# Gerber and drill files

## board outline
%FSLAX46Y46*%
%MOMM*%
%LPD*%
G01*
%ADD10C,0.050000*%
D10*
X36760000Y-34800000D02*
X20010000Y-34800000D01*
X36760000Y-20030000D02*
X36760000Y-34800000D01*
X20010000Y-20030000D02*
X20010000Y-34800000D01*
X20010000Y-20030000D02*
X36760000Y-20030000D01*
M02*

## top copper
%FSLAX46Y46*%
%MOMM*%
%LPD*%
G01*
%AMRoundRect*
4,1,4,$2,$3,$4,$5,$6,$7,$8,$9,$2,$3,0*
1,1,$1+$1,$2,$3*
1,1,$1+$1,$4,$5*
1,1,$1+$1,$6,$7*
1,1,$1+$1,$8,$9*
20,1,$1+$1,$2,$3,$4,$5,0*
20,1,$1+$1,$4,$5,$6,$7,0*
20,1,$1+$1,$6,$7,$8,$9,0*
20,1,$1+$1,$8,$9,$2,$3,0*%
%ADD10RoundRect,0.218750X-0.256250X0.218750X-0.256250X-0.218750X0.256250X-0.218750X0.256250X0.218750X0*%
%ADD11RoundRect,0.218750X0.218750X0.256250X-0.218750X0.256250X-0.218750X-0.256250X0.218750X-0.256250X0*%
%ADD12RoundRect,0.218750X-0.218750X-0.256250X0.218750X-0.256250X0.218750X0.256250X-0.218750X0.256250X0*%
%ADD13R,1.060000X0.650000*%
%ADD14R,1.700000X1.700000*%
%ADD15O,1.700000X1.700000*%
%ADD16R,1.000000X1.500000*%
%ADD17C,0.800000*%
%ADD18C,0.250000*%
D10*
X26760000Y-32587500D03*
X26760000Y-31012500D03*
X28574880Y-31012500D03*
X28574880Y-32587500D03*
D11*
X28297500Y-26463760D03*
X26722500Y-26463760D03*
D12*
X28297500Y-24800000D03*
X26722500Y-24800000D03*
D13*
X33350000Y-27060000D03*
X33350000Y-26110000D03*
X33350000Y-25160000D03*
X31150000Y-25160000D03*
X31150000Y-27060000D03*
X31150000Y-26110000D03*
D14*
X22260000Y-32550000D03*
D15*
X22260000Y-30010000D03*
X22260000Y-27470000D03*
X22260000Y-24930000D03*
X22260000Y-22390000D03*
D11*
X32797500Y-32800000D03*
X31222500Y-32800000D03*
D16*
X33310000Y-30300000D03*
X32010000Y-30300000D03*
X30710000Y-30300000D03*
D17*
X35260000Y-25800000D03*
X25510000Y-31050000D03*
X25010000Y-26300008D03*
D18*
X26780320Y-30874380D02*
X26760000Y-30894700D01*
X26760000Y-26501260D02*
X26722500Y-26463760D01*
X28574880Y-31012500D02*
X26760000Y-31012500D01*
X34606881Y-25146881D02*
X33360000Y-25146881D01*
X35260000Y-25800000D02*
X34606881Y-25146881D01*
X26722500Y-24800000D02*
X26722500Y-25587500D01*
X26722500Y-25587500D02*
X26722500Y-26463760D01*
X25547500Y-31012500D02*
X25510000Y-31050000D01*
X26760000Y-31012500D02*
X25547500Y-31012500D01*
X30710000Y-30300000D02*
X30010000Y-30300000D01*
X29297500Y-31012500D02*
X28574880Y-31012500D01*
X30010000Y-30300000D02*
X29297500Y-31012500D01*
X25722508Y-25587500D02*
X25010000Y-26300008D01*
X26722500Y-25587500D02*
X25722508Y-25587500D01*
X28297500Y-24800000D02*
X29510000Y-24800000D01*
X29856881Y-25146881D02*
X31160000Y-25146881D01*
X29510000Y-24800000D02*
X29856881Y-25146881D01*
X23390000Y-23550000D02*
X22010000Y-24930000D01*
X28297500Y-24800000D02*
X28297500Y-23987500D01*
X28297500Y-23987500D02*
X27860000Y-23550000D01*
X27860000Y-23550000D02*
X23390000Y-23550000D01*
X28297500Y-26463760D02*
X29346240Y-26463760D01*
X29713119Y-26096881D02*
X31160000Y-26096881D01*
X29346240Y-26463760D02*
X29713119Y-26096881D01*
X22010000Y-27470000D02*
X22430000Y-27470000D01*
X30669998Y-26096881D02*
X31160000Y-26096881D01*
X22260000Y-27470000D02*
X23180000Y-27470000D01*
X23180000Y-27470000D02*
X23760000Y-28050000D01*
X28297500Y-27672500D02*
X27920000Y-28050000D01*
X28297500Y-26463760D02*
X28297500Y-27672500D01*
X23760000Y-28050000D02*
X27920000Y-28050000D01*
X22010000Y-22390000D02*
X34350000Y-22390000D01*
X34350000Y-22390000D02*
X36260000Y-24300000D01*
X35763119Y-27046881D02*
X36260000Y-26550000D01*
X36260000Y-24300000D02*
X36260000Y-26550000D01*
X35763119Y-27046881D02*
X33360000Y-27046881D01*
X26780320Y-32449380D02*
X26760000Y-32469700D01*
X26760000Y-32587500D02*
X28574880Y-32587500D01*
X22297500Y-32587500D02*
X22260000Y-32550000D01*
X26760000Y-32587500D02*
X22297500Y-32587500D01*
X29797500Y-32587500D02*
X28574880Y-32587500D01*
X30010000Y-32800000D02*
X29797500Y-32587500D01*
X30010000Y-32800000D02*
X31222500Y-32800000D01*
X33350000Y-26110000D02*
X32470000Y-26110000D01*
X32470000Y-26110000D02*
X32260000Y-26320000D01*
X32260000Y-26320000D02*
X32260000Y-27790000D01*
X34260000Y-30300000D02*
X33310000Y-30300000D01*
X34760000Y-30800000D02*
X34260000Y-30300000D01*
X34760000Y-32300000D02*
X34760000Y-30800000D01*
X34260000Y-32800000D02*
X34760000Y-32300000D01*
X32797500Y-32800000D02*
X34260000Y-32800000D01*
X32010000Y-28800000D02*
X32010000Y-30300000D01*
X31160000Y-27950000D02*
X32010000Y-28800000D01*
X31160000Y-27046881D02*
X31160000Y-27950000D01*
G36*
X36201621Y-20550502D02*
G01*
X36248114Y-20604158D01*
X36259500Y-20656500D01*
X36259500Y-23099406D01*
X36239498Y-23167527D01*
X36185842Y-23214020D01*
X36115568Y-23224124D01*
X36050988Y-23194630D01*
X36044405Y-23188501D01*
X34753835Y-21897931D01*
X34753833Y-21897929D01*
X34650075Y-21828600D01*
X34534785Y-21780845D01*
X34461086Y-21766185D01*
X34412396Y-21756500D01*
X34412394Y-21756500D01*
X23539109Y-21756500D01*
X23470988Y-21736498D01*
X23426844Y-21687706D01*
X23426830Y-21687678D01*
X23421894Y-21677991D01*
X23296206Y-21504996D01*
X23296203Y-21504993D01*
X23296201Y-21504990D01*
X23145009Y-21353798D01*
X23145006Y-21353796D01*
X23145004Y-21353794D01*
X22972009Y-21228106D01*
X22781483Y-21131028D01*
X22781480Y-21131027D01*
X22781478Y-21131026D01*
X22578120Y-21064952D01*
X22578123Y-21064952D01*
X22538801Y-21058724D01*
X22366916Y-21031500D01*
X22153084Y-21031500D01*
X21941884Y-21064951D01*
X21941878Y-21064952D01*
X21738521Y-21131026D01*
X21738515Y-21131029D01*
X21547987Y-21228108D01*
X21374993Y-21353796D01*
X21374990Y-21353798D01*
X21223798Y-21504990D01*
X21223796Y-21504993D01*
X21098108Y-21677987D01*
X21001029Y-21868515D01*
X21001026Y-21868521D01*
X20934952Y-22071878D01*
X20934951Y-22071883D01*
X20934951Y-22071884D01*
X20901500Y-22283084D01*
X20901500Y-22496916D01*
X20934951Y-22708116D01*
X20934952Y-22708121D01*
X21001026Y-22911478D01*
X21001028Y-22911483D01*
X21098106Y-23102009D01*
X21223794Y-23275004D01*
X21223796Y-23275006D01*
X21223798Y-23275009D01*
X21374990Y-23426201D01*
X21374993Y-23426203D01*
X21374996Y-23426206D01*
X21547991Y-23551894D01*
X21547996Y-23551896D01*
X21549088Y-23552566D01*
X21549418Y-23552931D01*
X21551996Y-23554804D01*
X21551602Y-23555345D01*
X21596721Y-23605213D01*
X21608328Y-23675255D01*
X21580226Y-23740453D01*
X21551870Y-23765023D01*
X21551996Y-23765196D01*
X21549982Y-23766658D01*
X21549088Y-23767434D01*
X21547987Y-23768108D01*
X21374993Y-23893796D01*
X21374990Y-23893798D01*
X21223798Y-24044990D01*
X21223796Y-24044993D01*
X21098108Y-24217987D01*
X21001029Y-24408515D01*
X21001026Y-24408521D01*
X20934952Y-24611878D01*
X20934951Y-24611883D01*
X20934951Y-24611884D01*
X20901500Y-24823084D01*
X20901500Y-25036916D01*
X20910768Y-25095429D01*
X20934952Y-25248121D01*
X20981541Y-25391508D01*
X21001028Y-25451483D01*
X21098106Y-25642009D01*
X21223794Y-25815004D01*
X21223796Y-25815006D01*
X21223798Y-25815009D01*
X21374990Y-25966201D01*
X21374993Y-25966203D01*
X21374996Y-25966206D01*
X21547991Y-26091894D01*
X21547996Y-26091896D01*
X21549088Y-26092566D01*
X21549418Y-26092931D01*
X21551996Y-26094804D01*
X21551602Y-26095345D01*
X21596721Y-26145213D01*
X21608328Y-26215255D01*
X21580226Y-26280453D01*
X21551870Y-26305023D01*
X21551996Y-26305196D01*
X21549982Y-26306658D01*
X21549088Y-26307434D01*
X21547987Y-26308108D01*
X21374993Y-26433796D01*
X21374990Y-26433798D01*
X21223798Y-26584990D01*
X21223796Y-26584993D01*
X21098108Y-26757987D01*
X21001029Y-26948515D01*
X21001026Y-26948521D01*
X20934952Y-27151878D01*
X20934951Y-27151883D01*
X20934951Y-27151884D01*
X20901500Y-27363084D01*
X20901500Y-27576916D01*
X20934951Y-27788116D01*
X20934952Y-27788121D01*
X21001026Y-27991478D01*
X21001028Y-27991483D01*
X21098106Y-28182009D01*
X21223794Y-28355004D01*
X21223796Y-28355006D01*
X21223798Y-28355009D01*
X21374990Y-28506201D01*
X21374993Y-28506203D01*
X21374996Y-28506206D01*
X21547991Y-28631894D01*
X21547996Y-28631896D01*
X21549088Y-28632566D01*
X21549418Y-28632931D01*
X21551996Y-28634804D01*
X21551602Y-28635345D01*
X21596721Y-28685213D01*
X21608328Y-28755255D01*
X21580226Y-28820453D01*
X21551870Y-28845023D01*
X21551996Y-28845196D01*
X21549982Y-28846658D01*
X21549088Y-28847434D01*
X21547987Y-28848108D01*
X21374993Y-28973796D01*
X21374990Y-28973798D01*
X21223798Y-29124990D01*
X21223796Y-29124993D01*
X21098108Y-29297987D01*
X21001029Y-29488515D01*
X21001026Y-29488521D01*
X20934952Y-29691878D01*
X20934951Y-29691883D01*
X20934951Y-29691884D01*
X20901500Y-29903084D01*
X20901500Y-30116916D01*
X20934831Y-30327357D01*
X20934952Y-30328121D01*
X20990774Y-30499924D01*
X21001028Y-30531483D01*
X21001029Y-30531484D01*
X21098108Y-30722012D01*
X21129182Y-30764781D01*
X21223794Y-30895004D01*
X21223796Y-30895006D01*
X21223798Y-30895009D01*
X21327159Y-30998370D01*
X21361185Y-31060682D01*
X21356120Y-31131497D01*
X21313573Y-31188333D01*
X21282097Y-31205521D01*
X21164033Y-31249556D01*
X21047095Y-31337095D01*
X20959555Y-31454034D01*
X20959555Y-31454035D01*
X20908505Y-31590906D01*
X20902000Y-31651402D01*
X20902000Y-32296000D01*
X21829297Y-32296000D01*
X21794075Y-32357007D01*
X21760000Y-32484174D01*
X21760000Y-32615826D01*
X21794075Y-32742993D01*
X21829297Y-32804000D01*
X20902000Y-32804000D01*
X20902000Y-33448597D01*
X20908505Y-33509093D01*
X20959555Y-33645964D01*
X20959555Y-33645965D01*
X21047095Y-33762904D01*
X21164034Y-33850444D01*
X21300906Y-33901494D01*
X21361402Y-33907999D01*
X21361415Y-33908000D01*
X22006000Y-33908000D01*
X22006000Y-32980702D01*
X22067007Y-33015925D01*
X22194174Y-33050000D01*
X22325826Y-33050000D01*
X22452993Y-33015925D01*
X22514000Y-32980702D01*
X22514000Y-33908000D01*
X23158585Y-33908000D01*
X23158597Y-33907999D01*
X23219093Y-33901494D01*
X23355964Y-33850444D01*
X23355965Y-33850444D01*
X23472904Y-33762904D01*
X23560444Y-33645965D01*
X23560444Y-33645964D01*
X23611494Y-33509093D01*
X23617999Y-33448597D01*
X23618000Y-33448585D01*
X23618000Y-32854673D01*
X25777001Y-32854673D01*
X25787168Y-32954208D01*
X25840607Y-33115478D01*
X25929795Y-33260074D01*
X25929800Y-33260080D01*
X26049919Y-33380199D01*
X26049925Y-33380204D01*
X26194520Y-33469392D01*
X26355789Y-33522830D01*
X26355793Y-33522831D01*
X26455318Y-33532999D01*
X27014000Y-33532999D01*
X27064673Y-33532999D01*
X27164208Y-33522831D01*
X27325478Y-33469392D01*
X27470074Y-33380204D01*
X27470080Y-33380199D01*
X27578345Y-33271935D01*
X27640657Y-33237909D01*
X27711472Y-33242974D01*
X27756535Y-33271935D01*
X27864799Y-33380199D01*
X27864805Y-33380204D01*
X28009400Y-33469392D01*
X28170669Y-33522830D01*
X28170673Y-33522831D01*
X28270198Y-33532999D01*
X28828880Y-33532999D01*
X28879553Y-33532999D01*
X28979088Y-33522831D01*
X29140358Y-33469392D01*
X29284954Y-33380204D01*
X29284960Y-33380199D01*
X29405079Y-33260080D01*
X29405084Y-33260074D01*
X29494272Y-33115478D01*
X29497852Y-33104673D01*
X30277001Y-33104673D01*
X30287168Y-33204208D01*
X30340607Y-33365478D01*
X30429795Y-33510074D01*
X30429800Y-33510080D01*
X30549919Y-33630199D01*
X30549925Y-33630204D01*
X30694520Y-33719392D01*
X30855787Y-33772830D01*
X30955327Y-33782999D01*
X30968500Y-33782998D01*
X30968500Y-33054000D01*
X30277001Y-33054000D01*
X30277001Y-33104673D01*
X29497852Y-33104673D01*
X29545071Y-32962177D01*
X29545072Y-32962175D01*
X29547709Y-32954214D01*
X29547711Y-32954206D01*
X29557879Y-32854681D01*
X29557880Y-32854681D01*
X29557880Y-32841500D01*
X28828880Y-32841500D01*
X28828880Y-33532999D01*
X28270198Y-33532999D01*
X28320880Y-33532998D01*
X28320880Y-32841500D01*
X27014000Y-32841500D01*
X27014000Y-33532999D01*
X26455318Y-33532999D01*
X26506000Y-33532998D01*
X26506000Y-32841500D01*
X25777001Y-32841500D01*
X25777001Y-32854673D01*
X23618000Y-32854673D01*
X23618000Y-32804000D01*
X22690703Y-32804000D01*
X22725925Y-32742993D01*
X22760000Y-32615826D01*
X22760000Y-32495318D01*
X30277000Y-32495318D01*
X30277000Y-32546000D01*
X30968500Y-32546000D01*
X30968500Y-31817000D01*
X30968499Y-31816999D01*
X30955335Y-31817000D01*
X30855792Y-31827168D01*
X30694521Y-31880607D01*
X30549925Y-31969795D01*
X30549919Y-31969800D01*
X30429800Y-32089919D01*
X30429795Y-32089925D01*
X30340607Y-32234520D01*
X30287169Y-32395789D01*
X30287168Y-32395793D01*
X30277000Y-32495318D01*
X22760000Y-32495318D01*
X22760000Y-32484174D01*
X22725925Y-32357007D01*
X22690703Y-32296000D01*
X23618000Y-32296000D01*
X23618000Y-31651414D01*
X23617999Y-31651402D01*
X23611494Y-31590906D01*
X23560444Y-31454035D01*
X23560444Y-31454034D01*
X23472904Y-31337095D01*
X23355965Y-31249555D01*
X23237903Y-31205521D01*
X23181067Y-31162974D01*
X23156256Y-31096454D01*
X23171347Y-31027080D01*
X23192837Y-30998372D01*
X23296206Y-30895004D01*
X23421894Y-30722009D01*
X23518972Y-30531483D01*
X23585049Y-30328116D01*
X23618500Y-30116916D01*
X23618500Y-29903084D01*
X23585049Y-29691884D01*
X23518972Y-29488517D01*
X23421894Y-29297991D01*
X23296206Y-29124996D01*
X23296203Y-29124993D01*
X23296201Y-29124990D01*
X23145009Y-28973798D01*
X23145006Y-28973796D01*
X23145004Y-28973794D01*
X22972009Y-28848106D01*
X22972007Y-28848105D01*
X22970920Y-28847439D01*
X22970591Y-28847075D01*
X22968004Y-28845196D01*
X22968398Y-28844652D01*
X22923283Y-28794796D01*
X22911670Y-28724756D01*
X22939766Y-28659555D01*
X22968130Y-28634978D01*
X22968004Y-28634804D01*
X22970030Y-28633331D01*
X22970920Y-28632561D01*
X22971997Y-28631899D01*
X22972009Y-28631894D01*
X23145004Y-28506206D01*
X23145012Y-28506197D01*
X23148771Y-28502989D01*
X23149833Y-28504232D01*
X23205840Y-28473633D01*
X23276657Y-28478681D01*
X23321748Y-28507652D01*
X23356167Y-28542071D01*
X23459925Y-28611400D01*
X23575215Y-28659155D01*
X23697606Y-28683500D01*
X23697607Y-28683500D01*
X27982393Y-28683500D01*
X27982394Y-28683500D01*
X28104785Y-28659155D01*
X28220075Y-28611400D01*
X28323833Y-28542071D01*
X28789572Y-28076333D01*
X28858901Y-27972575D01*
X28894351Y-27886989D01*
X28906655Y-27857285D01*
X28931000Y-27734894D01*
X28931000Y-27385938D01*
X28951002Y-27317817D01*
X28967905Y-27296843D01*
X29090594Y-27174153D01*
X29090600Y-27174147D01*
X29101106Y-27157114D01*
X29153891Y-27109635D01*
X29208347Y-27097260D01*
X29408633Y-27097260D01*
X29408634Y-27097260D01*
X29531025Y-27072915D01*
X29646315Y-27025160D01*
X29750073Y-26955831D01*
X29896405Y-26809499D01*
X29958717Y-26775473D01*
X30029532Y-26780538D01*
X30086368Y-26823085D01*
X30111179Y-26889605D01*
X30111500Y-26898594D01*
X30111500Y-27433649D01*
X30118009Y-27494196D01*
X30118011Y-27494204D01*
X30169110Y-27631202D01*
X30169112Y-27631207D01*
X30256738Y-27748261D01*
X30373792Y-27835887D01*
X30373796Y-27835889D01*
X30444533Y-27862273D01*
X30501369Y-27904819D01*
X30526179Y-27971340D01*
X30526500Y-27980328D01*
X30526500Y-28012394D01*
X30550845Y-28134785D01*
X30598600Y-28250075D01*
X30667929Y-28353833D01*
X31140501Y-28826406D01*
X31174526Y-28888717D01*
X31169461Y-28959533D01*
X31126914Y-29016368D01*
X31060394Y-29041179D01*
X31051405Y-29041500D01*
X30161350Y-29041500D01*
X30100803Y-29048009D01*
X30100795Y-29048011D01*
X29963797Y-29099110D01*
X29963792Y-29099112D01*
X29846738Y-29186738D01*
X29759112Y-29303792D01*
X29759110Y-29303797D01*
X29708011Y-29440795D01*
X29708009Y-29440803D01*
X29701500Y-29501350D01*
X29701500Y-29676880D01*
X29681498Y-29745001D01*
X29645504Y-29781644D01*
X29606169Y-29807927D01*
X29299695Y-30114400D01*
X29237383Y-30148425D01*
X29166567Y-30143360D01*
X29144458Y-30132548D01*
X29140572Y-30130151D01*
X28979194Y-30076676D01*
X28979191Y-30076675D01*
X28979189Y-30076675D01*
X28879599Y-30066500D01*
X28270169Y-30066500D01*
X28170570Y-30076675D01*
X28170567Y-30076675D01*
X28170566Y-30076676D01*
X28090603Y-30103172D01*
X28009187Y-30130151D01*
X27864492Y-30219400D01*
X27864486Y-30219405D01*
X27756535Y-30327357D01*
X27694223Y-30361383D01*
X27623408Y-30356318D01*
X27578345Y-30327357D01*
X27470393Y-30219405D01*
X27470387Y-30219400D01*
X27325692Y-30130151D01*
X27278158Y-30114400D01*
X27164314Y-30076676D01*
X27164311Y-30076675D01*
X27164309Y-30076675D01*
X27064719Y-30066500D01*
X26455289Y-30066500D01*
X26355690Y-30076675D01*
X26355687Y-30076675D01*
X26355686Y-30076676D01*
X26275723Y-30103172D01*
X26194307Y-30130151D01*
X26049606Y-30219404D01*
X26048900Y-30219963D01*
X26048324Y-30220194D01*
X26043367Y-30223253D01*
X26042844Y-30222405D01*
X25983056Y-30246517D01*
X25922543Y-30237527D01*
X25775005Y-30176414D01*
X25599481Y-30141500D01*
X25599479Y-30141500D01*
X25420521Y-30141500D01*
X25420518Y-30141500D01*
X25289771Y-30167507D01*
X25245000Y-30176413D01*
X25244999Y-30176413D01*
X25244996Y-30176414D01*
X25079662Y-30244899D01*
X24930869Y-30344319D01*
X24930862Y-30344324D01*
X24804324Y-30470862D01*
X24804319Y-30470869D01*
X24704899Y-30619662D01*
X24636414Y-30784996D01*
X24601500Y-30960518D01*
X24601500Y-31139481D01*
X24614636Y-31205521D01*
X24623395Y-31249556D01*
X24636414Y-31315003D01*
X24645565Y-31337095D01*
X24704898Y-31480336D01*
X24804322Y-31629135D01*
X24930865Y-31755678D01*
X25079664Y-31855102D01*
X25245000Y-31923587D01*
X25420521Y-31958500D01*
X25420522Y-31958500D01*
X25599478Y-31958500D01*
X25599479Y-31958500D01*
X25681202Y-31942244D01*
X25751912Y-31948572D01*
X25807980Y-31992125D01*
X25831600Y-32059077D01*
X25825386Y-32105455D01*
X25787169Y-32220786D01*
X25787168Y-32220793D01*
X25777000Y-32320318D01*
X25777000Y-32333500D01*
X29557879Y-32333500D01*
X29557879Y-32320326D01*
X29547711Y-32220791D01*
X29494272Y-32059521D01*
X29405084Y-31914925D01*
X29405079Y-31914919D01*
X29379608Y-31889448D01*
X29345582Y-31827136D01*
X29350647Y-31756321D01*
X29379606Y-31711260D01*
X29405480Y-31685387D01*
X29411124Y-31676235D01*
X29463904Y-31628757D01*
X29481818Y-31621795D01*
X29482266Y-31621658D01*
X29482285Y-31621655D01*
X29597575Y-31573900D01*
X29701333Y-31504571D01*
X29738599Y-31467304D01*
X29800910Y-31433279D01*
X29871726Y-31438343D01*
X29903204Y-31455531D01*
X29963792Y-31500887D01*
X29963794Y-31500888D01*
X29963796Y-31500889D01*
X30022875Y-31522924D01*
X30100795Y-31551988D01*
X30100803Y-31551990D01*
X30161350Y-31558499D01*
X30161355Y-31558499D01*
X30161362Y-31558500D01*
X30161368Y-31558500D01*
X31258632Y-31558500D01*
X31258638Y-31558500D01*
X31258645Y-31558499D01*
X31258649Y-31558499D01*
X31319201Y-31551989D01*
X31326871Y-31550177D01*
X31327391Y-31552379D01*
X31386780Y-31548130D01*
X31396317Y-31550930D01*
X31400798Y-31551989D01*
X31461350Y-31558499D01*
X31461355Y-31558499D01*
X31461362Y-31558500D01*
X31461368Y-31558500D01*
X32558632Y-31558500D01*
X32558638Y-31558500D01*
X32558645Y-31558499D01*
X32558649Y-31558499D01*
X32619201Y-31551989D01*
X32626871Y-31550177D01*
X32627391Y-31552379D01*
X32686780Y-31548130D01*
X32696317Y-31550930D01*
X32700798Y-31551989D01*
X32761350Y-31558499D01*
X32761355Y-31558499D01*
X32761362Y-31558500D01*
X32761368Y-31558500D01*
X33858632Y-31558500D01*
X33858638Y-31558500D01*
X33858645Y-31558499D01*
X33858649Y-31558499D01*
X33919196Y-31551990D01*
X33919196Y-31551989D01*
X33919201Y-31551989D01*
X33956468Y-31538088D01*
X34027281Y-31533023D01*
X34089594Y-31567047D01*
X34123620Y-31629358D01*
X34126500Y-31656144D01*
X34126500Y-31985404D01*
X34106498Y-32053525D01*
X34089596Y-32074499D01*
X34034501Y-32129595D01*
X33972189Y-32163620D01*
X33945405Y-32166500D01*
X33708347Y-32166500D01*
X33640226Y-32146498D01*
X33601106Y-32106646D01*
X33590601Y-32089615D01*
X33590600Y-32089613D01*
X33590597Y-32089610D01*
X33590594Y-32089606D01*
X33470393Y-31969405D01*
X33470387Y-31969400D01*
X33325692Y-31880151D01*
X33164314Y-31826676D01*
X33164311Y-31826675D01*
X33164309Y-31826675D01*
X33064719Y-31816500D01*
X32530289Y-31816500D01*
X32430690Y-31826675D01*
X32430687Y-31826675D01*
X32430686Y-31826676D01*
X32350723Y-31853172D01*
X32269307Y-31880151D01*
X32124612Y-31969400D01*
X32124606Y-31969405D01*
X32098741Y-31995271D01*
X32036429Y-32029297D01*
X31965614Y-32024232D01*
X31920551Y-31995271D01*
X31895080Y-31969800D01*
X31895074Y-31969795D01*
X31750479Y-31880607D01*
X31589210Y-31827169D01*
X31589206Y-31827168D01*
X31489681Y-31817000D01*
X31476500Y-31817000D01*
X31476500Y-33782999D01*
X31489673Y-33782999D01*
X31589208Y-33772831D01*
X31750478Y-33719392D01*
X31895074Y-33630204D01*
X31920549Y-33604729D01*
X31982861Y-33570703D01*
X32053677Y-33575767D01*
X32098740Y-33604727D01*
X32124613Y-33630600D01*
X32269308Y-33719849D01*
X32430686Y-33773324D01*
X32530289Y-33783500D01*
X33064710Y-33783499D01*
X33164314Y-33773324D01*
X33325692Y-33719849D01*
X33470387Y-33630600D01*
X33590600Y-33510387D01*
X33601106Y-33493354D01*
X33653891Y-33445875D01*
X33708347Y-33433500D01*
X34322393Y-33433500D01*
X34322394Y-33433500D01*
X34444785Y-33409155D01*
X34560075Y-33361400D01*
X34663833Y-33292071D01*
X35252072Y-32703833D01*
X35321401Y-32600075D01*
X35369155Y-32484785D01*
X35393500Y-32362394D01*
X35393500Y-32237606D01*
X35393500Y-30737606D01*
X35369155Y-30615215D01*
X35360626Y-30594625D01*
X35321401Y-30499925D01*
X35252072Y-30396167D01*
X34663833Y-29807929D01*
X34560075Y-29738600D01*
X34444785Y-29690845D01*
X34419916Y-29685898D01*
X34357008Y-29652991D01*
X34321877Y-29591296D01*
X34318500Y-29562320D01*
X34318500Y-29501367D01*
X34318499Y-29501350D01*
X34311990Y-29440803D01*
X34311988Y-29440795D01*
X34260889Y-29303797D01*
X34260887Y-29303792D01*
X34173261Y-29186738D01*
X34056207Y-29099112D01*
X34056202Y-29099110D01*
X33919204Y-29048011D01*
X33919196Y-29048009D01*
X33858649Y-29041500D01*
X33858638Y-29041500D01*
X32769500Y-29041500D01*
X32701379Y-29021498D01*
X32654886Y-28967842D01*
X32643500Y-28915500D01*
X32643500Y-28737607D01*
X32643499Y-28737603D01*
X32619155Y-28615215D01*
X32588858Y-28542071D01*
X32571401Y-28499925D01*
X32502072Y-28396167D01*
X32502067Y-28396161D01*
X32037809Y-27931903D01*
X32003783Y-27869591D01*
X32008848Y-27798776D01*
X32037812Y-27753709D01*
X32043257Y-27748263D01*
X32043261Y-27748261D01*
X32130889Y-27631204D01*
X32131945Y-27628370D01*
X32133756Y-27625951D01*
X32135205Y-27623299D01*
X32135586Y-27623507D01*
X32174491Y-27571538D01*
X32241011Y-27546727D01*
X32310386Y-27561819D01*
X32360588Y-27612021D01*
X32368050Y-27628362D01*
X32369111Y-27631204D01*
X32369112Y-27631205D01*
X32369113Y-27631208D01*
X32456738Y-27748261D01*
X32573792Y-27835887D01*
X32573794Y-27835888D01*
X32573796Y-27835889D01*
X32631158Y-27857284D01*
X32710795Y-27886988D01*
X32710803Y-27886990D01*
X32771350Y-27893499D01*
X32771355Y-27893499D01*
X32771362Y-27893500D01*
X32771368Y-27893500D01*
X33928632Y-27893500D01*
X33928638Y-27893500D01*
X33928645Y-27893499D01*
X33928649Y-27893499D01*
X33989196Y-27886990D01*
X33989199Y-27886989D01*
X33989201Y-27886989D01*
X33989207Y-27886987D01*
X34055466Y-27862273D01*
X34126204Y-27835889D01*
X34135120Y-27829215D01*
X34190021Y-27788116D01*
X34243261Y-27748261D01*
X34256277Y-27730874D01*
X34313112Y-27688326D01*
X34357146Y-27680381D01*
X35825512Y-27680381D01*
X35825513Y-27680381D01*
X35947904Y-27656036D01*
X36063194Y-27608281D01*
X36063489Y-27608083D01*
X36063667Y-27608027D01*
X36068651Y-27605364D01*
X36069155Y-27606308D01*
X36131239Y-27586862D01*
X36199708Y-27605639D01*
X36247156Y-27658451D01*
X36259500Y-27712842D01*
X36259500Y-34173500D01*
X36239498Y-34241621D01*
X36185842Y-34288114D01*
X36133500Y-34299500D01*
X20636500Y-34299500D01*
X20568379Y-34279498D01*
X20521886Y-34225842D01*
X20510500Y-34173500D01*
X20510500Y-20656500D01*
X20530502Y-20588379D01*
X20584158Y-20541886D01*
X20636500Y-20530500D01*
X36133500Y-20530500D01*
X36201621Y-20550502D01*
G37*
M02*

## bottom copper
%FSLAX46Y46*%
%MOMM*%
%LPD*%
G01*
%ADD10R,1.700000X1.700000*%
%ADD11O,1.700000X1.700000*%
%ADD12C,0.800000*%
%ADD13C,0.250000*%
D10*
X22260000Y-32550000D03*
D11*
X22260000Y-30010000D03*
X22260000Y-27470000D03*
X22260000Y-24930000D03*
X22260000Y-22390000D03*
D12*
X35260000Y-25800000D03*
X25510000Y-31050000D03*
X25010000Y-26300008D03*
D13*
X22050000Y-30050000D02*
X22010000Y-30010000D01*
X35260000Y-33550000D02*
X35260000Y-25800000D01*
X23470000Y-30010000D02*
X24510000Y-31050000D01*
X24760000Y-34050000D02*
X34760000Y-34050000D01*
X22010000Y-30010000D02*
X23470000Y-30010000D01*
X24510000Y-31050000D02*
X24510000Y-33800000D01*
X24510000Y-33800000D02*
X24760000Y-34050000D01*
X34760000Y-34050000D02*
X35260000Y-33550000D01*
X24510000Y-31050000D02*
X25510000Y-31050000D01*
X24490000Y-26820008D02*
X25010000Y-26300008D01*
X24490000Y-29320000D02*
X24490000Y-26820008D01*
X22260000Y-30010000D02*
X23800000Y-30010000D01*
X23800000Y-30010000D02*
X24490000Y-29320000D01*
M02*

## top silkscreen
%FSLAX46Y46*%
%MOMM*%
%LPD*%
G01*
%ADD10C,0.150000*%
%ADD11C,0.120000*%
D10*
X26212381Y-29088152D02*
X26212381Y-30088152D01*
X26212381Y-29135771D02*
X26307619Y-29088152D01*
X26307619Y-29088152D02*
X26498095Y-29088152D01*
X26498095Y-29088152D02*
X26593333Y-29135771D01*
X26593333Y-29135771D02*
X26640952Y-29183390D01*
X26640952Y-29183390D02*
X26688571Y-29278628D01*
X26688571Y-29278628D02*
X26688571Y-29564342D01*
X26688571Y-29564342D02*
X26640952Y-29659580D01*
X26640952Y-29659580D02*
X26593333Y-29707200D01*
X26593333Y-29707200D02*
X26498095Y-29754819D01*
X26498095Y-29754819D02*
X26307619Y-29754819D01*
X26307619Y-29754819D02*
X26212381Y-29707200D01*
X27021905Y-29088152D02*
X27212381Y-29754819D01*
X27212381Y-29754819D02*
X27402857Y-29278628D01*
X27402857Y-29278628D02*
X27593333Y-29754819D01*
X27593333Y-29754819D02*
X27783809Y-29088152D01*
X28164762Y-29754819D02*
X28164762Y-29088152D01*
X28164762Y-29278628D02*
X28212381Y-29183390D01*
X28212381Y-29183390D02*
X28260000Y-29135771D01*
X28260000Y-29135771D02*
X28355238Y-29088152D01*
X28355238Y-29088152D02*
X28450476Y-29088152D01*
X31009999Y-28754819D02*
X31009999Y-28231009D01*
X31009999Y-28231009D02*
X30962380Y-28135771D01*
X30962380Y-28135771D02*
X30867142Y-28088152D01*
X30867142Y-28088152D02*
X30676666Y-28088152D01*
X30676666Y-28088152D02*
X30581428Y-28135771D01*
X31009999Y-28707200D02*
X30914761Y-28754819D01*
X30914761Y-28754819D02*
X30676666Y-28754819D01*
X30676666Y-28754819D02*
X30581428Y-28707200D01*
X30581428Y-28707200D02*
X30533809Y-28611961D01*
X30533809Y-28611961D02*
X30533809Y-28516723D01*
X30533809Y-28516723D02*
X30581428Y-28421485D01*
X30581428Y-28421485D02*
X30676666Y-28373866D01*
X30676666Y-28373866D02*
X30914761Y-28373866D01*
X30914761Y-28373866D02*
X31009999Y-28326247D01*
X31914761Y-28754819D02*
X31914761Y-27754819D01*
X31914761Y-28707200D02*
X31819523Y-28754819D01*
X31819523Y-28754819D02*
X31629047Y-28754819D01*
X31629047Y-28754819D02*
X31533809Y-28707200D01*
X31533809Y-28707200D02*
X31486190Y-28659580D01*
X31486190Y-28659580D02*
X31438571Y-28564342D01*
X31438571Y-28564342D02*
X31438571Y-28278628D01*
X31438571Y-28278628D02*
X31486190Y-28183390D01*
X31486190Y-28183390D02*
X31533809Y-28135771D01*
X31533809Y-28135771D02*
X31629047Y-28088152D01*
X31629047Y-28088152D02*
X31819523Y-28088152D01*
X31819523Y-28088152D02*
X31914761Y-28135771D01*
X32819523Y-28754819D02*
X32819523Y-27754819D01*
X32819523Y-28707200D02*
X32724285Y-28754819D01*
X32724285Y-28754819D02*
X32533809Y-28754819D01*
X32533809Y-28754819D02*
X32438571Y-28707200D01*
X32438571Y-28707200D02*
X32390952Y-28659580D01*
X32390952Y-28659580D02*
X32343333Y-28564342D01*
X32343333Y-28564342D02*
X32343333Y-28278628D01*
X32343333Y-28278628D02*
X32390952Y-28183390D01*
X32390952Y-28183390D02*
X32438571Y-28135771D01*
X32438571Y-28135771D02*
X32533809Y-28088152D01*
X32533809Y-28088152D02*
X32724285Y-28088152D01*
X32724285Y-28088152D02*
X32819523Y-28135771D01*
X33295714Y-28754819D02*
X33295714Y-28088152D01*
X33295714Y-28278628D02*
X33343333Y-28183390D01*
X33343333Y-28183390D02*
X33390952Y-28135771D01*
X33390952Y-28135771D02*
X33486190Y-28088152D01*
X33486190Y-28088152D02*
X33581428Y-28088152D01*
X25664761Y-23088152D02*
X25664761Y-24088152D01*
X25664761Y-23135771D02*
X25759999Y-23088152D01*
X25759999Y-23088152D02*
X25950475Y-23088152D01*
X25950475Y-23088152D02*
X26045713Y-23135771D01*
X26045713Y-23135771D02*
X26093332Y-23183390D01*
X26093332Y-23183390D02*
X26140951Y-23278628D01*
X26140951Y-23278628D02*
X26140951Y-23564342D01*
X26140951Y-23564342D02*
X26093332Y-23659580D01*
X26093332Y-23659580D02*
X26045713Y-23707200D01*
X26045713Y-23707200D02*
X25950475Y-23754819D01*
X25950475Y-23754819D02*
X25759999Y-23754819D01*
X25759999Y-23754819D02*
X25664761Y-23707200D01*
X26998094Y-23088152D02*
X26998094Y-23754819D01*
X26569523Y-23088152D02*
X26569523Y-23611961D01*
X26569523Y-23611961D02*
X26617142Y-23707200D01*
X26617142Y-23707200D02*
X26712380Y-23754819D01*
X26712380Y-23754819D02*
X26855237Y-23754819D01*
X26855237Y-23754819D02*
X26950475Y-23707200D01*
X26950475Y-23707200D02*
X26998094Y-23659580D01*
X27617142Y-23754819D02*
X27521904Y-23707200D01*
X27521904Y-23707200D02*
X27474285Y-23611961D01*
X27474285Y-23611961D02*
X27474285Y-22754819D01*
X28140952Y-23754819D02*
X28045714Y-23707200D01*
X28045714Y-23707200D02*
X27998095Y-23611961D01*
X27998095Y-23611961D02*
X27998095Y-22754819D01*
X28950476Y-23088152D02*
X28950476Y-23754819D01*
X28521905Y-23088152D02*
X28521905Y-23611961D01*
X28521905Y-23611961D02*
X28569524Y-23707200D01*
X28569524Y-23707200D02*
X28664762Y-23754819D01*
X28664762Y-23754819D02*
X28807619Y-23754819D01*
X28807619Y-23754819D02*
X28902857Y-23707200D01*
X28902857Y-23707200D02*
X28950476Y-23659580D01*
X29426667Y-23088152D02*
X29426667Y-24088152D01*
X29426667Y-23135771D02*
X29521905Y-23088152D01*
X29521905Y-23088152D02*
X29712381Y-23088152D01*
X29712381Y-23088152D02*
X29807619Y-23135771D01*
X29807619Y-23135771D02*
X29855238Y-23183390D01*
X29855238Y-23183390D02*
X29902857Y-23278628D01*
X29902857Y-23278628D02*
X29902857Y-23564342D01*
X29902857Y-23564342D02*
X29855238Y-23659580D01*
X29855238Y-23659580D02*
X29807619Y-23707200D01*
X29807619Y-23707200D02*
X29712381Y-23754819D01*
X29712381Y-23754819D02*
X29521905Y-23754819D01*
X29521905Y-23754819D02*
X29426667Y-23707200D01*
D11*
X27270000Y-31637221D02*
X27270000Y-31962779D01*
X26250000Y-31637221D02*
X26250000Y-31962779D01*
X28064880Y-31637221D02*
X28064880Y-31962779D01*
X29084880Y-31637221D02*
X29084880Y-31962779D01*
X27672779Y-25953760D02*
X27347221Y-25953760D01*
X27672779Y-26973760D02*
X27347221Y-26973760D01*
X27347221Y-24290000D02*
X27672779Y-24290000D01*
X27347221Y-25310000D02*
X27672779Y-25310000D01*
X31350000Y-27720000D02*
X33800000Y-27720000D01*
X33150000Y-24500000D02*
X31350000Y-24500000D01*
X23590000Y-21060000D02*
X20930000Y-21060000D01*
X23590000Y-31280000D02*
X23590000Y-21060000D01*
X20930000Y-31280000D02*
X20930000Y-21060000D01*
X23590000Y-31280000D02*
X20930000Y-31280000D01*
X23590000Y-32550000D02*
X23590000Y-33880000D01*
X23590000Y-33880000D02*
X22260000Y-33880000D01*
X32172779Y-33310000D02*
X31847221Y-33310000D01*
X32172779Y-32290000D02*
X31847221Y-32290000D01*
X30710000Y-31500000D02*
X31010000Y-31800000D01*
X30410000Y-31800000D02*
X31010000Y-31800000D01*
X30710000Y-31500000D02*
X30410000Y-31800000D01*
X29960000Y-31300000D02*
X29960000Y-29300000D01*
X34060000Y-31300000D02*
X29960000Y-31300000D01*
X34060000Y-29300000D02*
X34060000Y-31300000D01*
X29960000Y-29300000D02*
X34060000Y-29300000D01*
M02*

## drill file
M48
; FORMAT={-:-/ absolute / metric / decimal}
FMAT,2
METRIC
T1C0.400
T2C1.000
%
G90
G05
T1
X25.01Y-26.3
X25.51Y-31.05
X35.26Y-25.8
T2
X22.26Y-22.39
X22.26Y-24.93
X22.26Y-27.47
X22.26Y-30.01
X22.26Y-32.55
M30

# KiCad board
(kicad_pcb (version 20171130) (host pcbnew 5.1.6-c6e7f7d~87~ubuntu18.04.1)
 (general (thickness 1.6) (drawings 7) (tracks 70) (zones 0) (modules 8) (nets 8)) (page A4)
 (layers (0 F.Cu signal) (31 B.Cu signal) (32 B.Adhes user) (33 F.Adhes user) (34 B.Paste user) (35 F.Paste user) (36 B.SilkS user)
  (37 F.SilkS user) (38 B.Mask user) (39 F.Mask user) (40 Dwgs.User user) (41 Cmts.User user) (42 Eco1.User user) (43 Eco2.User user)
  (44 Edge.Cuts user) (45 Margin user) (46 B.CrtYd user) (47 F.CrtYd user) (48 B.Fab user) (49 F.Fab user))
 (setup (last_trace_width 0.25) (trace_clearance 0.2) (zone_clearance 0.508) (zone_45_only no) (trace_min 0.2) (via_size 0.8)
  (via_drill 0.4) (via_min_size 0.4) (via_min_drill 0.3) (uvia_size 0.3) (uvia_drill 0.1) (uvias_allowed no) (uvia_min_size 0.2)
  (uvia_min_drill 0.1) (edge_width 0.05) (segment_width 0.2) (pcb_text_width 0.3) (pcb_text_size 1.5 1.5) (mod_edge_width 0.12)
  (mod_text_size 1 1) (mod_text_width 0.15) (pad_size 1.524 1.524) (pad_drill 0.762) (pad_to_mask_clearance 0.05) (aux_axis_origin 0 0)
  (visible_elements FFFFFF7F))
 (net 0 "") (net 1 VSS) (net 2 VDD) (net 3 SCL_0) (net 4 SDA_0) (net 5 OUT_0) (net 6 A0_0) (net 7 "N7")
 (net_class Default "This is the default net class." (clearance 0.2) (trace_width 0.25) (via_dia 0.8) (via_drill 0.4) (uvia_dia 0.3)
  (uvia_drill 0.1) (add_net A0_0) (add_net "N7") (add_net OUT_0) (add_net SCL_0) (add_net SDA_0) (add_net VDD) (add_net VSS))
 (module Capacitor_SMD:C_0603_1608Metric (layer F.Cu) (at 26.76 31.8 270)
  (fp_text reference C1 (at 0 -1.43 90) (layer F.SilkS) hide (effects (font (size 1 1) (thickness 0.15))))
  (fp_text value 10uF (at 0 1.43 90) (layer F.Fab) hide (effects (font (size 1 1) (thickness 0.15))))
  (fp_line (start -0.162779 -0.51) (end 0.162779 -0.51) (layer F.SilkS) (width 0.12))
  (fp_line (start -0.162779 0.51) (end 0.162779 0.51) (layer F.SilkS) (width 0.12))
  (pad 2 smd roundrect (at 0.7875 0 270) (size 0.875 0.95) (layers F.Cu F.Paste F.Mask) (roundrect_rratio 0.25) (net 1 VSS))
  (pad 1 smd roundrect (at -0.7875 0 270) (size 0.875 0.95) (layers F.Cu F.Paste F.Mask) (roundrect_rratio 0.25) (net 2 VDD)))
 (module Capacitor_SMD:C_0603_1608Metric (layer F.Cu) (at 28.57488 31.8 270)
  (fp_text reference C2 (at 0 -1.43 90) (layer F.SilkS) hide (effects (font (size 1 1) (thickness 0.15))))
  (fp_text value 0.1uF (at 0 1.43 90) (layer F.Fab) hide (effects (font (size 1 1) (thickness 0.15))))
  (fp_line (start -0.162779 0.51) (end 0.162779 0.51) (layer F.SilkS) (width 0.12))
  (fp_line (start -0.162779 -0.51) (end 0.162779 -0.51) (layer F.SilkS) (width 0.12))
  (pad 1 smd roundrect (at -0.7875 0 270) (size 0.875 0.95) (layers F.Cu F.Paste F.Mask) (roundrect_rratio 0.25) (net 2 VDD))
  (pad 2 smd roundrect (at 0.7875 0 270) (size 0.875 0.95) (layers F.Cu F.Paste F.Mask) (roundrect_rratio 0.25) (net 1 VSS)))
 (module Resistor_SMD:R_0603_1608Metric (layer F.Cu) (at 27.51 26.46376 180)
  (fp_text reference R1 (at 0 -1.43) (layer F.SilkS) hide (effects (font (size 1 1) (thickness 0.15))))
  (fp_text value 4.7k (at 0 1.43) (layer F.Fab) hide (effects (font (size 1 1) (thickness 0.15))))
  (fp_line (start -0.162779 0.51) (end 0.162779 0.51) (layer F.SilkS) (width 0.12))
  (fp_line (start -0.162779 -0.51) (end 0.162779 -0.51) (layer F.SilkS) (width 0.12))
  (pad 1 smd roundrect (at -0.7875 0 180) (size 0.875 0.95) (layers F.Cu F.Paste F.Mask) (roundrect_rratio 0.25) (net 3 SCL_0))
  (pad 2 smd roundrect (at 0.7875 0 180) (size 0.875 0.95) (layers F.Cu F.Paste F.Mask) (roundrect_rratio 0.25) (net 2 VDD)))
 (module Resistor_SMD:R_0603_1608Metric (layer F.Cu) (at 27.51 24.8)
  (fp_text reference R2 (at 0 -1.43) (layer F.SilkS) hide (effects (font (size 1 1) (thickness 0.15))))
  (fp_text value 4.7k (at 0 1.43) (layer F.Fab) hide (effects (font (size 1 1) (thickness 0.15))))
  (fp_line (start -0.162779 -0.51) (end 0.162779 -0.51) (layer F.SilkS) (width 0.12))
  (fp_line (start -0.162779 0.51) (end 0.162779 0.51) (layer F.SilkS) (width 0.12))
  (pad 2 smd roundrect (at 0.7875 0) (size 0.875 0.95) (layers F.Cu F.Paste F.Mask) (roundrect_rratio 0.25) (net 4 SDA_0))
  (pad 1 smd roundrect (at -0.7875 0) (size 0.875 0.95) (layers F.Cu F.Paste F.Mask) (roundrect_rratio 0.25) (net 2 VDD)))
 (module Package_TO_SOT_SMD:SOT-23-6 (layer F.Cu) (at 32.25 26.11 180)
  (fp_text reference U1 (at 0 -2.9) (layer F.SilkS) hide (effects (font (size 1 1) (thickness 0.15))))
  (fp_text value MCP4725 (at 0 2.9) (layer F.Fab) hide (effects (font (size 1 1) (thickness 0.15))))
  (fp_line (start 0.9 -1.61) (end -1.55 -1.61) (layer F.SilkS) (width 0.12))
  (fp_line (start -0.9 1.61) (end 0.9 1.61) (layer F.SilkS) (width 0.12))
  (pad 1 smd rect (at -1.1 -0.95 180) (size 1.06 0.65) (layers F.Cu F.Paste F.Mask) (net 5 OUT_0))
  (pad 2 smd rect (at -1.1 0 180) (size 1.06 0.65) (layers F.Cu F.Paste F.Mask) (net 1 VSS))
  (pad 3 smd rect (at -1.1 0.95 180) (size 1.06 0.65) (layers F.Cu F.Paste F.Mask) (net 2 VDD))
  (pad 4 smd rect (at 1.1 0.95 180) (size 1.06 0.65) (layers F.Cu F.Paste F.Mask) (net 4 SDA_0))
  (pad 6 smd rect (at 1.1 -0.95 180) (size 1.06 0.65) (layers F.Cu F.Paste F.Mask) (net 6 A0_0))
  (pad 5 smd rect (at 1.1 0 180) (size 1.06 0.65) (layers F.Cu F.Paste F.Mask) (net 3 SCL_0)))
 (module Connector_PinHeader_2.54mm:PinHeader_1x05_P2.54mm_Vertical (layer F.Cu) (at 22.26 32.55 180)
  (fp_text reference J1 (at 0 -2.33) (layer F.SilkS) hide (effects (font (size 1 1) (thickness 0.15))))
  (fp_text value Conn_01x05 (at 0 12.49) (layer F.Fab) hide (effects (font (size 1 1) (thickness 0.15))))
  (fp_line (start -1.33 11.49) (end 1.33 11.49) (layer F.SilkS) (width 0.12))
  (fp_line (start -1.33 1.27) (end -1.33 11.49) (layer F.SilkS) (width 0.12))
  (fp_line (start 1.33 1.27) (end 1.33 11.49) (layer F.SilkS) (width 0.12))
  (fp_line (start -1.33 1.27) (end 1.33 1.27) (layer F.SilkS) (width 0.12))
  (fp_line (start -1.33 0) (end -1.33 -1.33) (layer F.SilkS) (width 0.12))
  (fp_line (start -1.33 -1.33) (end 0 -1.33) (layer F.SilkS) (width 0.12))
  (pad 1 thru_hole rect (at 0 0 180) (size 1.7 1.7) (drill 1) (layers *.Cu *.Mask) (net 1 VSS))
  (pad 2 thru_hole oval (at 0 2.54 180) (size 1.7 1.7) (drill 1) (layers *.Cu *.Mask) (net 2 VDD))
  (pad 3 thru_hole oval (at 0 5.08 180) (size 1.7 1.7) (drill 1) (layers *.Cu *.Mask) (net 3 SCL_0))
  (pad 4 thru_hole oval (at 0 7.62 180) (size 1.7 1.7) (drill 1) (layers *.Cu *.Mask) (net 4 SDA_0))
  (pad 5 thru_hole oval (at 0 10.16 180) (size 1.7 1.7) (drill 1) (layers *.Cu *.Mask) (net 5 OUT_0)))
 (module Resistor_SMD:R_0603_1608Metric (layer F.Cu) (at 32.01 32.8 180)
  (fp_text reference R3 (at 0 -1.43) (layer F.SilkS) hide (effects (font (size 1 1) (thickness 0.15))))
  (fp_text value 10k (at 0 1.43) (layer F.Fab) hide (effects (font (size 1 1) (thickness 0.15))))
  (fp_line (start -0.162779 -0.51) (end 0.162779 -0.51) (layer F.SilkS) (width 0.12))
  (fp_line (start -0.162779 0.51) (end 0.162779 0.51) (layer F.SilkS) (width 0.12))
  (pad 1 smd roundrect (at -0.7875 0 180) (size 0.875 0.95) (layers F.Cu F.Paste F.Mask) (roundrect_rratio 0.25) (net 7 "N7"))
  (pad 2 smd roundrect (at 0.7875 0 180) (size 0.875 0.95) (layers F.Cu F.Paste F.Mask) (roundrect_rratio 0.25) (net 1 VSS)))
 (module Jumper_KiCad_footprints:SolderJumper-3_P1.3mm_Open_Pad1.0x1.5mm (layer F.Cu) (at 32.01 30.3)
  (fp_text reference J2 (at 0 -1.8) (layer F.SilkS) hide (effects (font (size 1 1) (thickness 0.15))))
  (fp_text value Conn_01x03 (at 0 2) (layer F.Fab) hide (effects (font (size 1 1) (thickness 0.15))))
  (fp_line (start -1.3 1.2) (end -1 1.5) (layer F.SilkS) (width 0.12))
  (fp_line (start -1.6 1.5) (end -1 1.5) (layer F.SilkS) (width 0.12))
  (fp_line (start -1.3 1.2) (end -1.6 1.5) (layer F.SilkS) (width 0.12))
  (fp_line (start -2.05 1) (end -2.05 -1) (layer F.SilkS) (width 0.12))
  (fp_line (start 2.05 1) (end -2.05 1) (layer F.SilkS) (width 0.12))
  (fp_line (start 2.05 -1) (end 2.05 1) (layer F.SilkS) (width 0.12))
  (fp_line (start -2.05 -1) (end 2.05 -1) (layer F.SilkS) (width 0.12))
  (pad 3 smd rect (at 1.3 0) (size 1 1.5) (layers F.Cu F.Mask) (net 7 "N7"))
  (pad 2 smd rect (at 0 0) (size 1 1.5) (layers F.Cu F.Mask) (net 6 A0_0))
  (pad 1 smd rect (at -1.3 0) (size 1 1.5) (layers F.Cu F.Mask) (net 2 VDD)))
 (gr_line (start 36.76 34.8) (end 20.01 34.8) (layer Edge.Cuts) (width 0.05))
 (gr_line (start 36.76 20.03) (end 36.76 34.8) (layer Edge.Cuts) (width 0.05))
 (gr_line (start 20.01 20.03) (end 20.01 34.8) (layer Edge.Cuts) (width 0.05))
 (gr_line (start 20.01 20.03) (end 36.76 20.03) (layer Edge.Cuts) (width 0.05))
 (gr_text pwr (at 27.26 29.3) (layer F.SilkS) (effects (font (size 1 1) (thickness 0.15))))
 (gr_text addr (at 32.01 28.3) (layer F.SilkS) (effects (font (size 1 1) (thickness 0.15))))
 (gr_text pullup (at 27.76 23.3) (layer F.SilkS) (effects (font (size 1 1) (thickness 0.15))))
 (segment (start 26.78032 30.87438) (end 26.76 30.8947) (width 0.25) (layer F.Cu) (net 2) (status 30))
 (segment (start 26.76 26.50126) (end 26.7225 26.46376) (width 0.25) (layer F.Cu) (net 2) (status 30))
 (segment (start 28.57488 31.0125) (end 26.76 31.0125) (width 0.25) (layer F.Cu) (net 2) (status 30))
 (via (at 35.26 25.8) (size 0.8) (drill 0.4) (layers F.Cu B.Cu) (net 2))
 (segment (start 34.606881 25.146881) (end 33.36 25.146881) (width 0.25) (layer F.Cu) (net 2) (status 20))
 (segment (start 35.26 25.8) (end 34.606881 25.146881) (width 0.25) (layer F.Cu) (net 2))
 (segment (start 26.7225 24.8) (end 26.7225 25.5875) (width 0.25) (layer F.Cu) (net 2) (status 10))
 (segment (start 26.7225 25.5875) (end 26.7225 26.46376) (width 0.25) (layer F.Cu) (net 2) (status 20))
 (segment (start 22.05 30.05) (end 22.01 30.01) (width 0.25) (layer B.Cu) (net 2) (status 30))
 (segment (start 35.26 33.55) (end 35.26 25.8) (width 0.25) (layer B.Cu) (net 2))
 (segment (start 23.47 30.01) (end 24.51 31.05) (width 0.25) (layer B.Cu) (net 2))
 (segment (start 24.76 34.05) (end 34.76 34.05) (width 0.25) (layer B.Cu) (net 2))
 (segment (start 22.01 30.01) (end 23.47 30.01) (width 0.25) (layer B.Cu) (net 2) (status 10))
 (segment (start 24.51 31.05) (end 24.51 33.8) (width 0.25) (layer B.Cu) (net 2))
 (segment (start 24.51 33.8) (end 24.76 34.05) (width 0.25) (layer B.Cu) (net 2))
 (segment (start 34.76 34.05) (end 35.26 33.55) (width 0.25) (layer B.Cu) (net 2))
 (segment (start 25.5475 31.0125) (end 25.51 31.05) (width 0.25) (layer F.Cu) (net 2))
 (segment (start 26.76 31.0125) (end 25.5475 31.0125) (width 0.25) (layer F.Cu) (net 2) (status 10))
 (via (at 25.51 31.05) (size 0.8) (drill 0.4) (layers F.Cu B.Cu) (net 2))
 (segment (start 24.51 31.05) (end 25.51 31.05) (width 0.25) (layer B.Cu) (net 2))
 (segment (start 30.71 30.3) (end 30.01 30.3) (width 0.25) (layer F.Cu) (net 2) (status 10))
 (segment (start 29.2975 31.0125) (end 28.57488 31.0125) (width 0.25) (layer F.Cu) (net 2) (status 20))
 (segment (start 30.01 30.3) (end 29.2975 31.0125) (width 0.25) (layer F.Cu) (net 2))
 (via (at 25.01 26.300008) (size 0.8) (drill 0.4) (layers F.Cu B.Cu) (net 2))
 (segment (start 25.722508 25.5875) (end 25.01 26.300008) (width 0.25) (layer F.Cu) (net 2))
 (segment (start 26.7225 25.5875) (end 25.722508 25.5875) (width 0.25) (layer F.Cu) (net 2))
 (segment (start 24.49 26.820008) (end 25.01 26.300008) (width 0.25) (layer B.Cu) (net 2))
 (segment (start 24.49 29.32) (end 24.49 26.820008) (width 0.25) (layer B.Cu) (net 2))
 (segment (start 22.26 30.01) (end 23.8 30.01) (width 0.25) (layer B.Cu) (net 2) (status 10))
 (segment (start 23.8 30.01) (end 24.49 29.32) (width 0.25) (layer B.Cu) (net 2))
 (segment (start 28.2975 24.8) (end 29.51 24.8) (width 0.25) (layer F.Cu) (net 4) (status 10))
 (segment (start 29.856881 25.146881) (end 31.16 25.146881) (width 0.25) (layer F.Cu) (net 4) (status 20))
 (segment (start 29.51 24.8) (end 29.856881 25.146881) (width 0.25) (layer F.Cu) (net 4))
 (segment (start 23.39 23.55) (end 22.01 24.93) (width 0.25) (layer F.Cu) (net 4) (status 20))
 (segment (start 28.2975 24.8) (end 28.2975 23.9875) (width 0.25) (layer F.Cu) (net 4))
 (segment (start 28.2975 23.9875) (end 27.86 23.55) (width 0.25) (layer F.Cu) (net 4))
 (segment (start 27.86 23.55) (end 23.39 23.55) (width 0.25) (layer F.Cu) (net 4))
 (segment (start 28.2975 26.46376) (end 29.34624 26.46376) (width 0.25) (layer F.Cu) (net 3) (status 10))
 (segment (start 29.713119 26.096881) (end 31.16 26.096881) (width 0.25) (layer F.Cu) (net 3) (status 20))
 (segment (start 29.34624 26.46376) (end 29.713119 26.096881) (width 0.25) (layer F.Cu) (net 3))
 (segment (start 22.01 27.47) (end 22.43 27.47) (width 0.25) (layer F.Cu) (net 3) (status 30))
 (segment (start 30.669998 26.096881) (end 31.16 26.096881) (width 0.25) (layer F.Cu) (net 3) (status 30))
 (segment (start 22.26 27.47) (end 23.18 27.47) (width 0.25) (layer F.Cu) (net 3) (status 10))
 (segment (start 23.18 27.47) (end 23.76 28.05) (width 0.25) (layer F.Cu) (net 3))
 (segment (start 28.2975 27.6725) (end 27.92 28.05) (width 0.25) (layer F.Cu) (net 3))
 (segment (start 28.2975 26.46376) (end 28.2975 27.6725) (width 0.25) (layer F.Cu) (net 3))
 (segment (start 23.76 28.05) (end 27.92 28.05) (width 0.25) (layer F.Cu) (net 3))
 (segment (start 22.01 22.39) (end 34.35 22.39) (width 0.25) (layer F.Cu) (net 5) (status 10))
 (segment (start 34.35 22.39) (end 36.26 24.3) (width 0.25) (layer F.Cu) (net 5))
 (segment (start 35.763119 27.046881) (end 36.26 26.55) (width 0.25) (layer F.Cu) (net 5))
 (segment (start 36.26 24.3) (end 36.26 26.55) (width 0.25) (layer F.Cu) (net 5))
 (segment (start 35.763119 27.046881) (end 33.36 27.046881) (width 0.25) (layer F.Cu) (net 5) (status 20))
 (segment (start 26.78032 32.44938) (end 26.76 32.4697) (width 0.25) (layer F.Cu) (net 1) (status 30))
 (segment (start 26.76 32.5875) (end 28.57488 32.5875) (width 0.25) (layer F.Cu) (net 1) (status 30))
 (segment (start 22.2975 32.5875) (end 22.26 32.55) (width 0.25) (layer F.Cu) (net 1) (status 30))
 (segment (start 26.76 32.5875) (end 22.2975 32.5875) (width 0.25) (layer F.Cu) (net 1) (status 30))
 (segment (start 29.7975 32.5875) (end 28.57488 32.5875) (width 0.25) (layer F.Cu) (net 1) (status 20))
 (segment (start 30.01 32.8) (end 29.7975 32.5875) (width 0.25) (layer F.Cu) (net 1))
 (segment (start 30.01 32.8) (end 31.2225 32.8) (width 0.25) (layer F.Cu) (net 1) (status 20))
 (segment (start 33.35 26.11) (end 32.47 26.11) (width 0.25) (layer F.Cu) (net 1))
 (segment (start 32.47 26.11) (end 32.26 26.32) (width 0.25) (layer F.Cu) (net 1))
 (segment (start 32.26 26.32) (end 32.26 27.79) (width 0.25) (layer F.Cu) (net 1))
 (segment (start 34.26 30.3) (end 33.31 30.3) (width 0.25) (layer F.Cu) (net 7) (status 20))
 (segment (start 34.76 30.8) (end 34.26 30.3) (width 0.25) (layer F.Cu) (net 7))
 (segment (start 34.76 32.3) (end 34.76 30.8) (width 0.25) (layer F.Cu) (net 7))
 (segment (start 34.26 32.8) (end 34.76 32.3) (width 0.25) (layer F.Cu) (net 7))
 (segment (start 32.7975 32.8) (end 34.26 32.8) (width 0.25) (layer F.Cu) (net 7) (status 10))
 (segment (start 32.01 28.8) (end 32.01 30.3) (width 0.25) (layer F.Cu) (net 6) (status 20))
 (segment (start 31.16 27.95) (end 32.01 28.8) (width 0.25) (layer F.Cu) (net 6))
 (segment (start 31.16 27.046881) (end 31.16 27.95) (width 0.25) (layer F.Cu) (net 6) (status 10))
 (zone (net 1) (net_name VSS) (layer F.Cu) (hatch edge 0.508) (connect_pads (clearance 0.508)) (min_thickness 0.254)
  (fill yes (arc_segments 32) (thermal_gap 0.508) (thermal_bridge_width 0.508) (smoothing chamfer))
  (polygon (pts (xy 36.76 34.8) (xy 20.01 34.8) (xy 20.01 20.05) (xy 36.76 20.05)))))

